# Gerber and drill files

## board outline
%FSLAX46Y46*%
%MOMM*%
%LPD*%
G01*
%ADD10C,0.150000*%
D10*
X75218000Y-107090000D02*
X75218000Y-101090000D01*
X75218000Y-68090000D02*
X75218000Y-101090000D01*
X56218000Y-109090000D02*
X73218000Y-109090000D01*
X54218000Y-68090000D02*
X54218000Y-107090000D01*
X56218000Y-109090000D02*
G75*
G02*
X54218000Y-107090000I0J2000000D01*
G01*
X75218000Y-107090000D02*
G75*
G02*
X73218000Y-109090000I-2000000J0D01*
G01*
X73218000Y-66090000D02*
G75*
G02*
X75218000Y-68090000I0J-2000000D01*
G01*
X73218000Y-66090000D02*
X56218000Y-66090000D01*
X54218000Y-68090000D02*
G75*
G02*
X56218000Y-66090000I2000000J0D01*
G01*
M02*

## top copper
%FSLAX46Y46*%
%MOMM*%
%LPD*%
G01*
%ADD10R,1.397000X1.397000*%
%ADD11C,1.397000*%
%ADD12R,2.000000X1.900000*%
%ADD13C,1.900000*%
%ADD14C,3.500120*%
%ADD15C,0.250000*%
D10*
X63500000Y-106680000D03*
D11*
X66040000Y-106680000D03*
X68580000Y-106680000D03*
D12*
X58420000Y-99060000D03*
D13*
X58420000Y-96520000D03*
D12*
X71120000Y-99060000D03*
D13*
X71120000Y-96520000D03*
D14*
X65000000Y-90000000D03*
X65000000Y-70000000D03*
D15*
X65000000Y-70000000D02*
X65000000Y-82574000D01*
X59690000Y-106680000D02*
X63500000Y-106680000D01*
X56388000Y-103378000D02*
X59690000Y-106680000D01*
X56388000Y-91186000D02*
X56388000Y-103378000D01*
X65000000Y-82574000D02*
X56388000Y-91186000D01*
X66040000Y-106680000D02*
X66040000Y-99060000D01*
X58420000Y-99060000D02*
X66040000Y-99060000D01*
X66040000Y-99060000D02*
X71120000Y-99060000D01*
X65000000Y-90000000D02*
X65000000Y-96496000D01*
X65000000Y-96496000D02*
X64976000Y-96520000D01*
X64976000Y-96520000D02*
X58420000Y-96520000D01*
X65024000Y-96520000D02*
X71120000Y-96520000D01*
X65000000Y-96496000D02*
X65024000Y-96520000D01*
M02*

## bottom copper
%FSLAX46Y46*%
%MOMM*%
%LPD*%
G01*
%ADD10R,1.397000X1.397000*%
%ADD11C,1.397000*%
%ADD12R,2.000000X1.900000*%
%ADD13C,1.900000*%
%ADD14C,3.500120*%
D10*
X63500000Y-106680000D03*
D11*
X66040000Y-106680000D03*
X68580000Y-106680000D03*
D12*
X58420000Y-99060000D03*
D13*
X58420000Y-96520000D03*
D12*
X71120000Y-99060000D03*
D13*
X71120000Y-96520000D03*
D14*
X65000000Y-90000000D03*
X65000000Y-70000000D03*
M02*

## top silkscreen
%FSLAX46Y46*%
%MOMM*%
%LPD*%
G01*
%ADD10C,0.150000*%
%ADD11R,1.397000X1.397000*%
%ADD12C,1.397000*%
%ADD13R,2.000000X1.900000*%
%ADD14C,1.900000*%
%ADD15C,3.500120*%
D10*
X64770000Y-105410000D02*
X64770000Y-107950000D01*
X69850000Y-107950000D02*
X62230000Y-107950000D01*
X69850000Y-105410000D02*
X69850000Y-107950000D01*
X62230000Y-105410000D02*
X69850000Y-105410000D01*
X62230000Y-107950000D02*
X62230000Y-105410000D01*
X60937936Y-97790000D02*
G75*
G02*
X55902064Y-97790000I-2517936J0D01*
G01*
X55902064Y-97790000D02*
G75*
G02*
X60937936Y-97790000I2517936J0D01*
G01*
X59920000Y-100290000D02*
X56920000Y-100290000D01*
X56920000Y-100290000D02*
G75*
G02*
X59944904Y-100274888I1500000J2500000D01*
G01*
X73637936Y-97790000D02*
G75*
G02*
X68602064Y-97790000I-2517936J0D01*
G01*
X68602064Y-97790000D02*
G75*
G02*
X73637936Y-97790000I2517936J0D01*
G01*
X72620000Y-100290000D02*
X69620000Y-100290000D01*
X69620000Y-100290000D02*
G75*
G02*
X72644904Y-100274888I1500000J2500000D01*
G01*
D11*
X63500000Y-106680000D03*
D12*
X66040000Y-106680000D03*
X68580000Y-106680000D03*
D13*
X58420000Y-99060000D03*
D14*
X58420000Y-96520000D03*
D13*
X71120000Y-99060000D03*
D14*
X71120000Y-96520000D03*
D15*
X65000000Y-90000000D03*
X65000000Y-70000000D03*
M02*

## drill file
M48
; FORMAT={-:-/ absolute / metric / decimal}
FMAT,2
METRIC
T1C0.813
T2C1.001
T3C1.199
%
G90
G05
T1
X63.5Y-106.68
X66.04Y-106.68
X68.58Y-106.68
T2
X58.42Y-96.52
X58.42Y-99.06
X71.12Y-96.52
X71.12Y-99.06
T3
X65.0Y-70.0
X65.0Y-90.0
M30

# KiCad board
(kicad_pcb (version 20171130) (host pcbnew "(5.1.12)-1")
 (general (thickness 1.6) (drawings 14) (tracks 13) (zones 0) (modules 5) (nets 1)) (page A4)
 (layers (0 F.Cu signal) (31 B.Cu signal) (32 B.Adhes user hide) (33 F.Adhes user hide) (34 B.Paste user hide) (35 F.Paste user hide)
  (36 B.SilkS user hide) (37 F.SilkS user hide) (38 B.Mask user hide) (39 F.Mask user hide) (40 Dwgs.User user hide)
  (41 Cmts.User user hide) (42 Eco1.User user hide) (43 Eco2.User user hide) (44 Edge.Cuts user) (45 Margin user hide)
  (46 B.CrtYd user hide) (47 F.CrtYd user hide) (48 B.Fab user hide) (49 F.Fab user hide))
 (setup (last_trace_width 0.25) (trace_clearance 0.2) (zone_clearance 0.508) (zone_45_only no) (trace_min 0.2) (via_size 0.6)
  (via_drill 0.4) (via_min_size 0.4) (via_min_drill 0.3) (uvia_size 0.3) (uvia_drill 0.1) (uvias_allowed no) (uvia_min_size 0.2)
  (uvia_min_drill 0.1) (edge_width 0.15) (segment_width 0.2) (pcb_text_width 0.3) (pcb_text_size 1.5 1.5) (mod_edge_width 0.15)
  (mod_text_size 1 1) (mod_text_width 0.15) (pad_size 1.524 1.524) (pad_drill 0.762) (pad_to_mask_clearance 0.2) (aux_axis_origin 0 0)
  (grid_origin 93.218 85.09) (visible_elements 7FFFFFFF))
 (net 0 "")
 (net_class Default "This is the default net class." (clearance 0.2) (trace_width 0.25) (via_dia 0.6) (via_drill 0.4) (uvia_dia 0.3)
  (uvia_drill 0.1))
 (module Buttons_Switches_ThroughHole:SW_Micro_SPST (layer F.Cu) (at 66.04 106.68)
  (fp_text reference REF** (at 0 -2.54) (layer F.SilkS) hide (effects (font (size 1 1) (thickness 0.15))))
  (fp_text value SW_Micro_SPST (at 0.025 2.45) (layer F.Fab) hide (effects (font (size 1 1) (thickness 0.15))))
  (fp_line (start -1.27 -1.27) (end -1.27 1.27) (layer F.SilkS) (width 0.15))
  (fp_line (start 3.81 1.27) (end -3.81 1.27) (layer F.SilkS) (width 0.15))
  (fp_line (start 3.81 -1.27) (end 3.81 1.27) (layer F.SilkS) (width 0.15))
  (fp_line (start -3.81 -1.27) (end 3.81 -1.27) (layer F.SilkS) (width 0.15))
  (fp_line (start -3.81 1.27) (end -3.81 -1.27) (layer F.SilkS) (width 0.15))
  (pad 1 thru_hole rect (at -2.54 0) (size 1.397 1.397) (drill 0.8128) (layers *.Cu *.Mask F.SilkS))
  (pad 2 thru_hole circle (at 0 0) (size 1.397 1.397) (drill 0.8128) (layers *.Cu *.Mask F.SilkS))
  (pad 3 thru_hole circle (at 2.54 0) (size 1.397 1.397) (drill 0.8128) (layers *.Cu *.Mask F.SilkS)))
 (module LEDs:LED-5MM (layer F.Cu) (at 58.42 99.06 90)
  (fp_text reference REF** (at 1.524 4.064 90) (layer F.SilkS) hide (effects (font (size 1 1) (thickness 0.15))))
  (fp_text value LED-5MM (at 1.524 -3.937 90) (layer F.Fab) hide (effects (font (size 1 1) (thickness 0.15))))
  (fp_circle (center 1.27 0) (end 0.97 -2.5) (layer F.SilkS) (width 0.15))
  (fp_line (start -1.23 1.5) (end -1.23 -1.5) (layer F.SilkS) (width 0.15))
  (fp_arc (start 1.27 0) (end -1.23 -1.5) (angle 297.5) (layer F.SilkS) (width 0.15))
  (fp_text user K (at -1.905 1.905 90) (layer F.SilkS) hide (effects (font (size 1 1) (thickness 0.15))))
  (pad 1 thru_hole rect (at 0 0 180) (size 2 1.9) (drill 1.00076) (layers *.Cu *.Mask F.SilkS))
  (pad 2 thru_hole circle (at 2.54 0 90) (size 1.9 1.9) (drill 1.00076) (layers *.Cu *.Mask F.SilkS)))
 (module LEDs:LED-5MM (layer F.Cu) (at 71.12 99.06 90)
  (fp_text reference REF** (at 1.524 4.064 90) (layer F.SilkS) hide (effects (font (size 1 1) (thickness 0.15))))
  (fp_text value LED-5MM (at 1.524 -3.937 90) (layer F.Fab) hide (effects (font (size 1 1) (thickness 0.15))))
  (fp_circle (center 1.27 0) (end 0.97 -2.5) (layer F.SilkS) (width 0.15))
  (fp_line (start -1.23 1.5) (end -1.23 -1.5) (layer F.SilkS) (width 0.15))
  (fp_arc (start 1.27 0) (end -1.23 -1.5) (angle 297.5) (layer F.SilkS) (width 0.15))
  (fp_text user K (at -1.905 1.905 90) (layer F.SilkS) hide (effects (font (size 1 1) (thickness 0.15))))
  (pad 1 thru_hole rect (at 0 0 180) (size 2 1.9) (drill 1.00076) (layers *.Cu *.Mask F.SilkS))
  (pad 2 thru_hole circle (at 2.54 0 90) (size 1.9 1.9) (drill 1.00076) (layers *.Cu *.Mask F.SilkS)))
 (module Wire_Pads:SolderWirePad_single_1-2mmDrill (layer F.Cu) (at 65 90)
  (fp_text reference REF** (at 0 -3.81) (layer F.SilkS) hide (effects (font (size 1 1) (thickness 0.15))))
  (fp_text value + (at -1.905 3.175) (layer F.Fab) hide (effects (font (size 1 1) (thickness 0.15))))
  (pad 1 thru_hole circle (at 0 0) (size 3.50012 3.50012) (drill 1.19888) (layers *.Cu *.Mask F.SilkS)))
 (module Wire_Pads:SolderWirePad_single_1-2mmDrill (layer F.Cu) (at 65 70)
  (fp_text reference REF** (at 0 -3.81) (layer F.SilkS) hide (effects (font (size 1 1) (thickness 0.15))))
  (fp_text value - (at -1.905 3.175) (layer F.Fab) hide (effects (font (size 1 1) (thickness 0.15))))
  (pad 1 thru_hole circle (at 0 0) (size 3.50012 3.50012) (drill 1.19888) (layers *.Cu *.Mask F.SilkS)))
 (gr_line (start 75.218 107.09) (end 75.218 101.09) (angle 90) (layer Edge.Cuts) (width 0.15))
 (gr_line (start 75.218 68.09) (end 75.218 101.09) (angle 90) (layer Edge.Cuts) (width 0.15))
 (gr_line (start 56.218 109.09) (end 73.218 109.09) (angle 90) (layer Edge.Cuts) (width 0.15))
 (gr_line (start 54.218 68.09) (end 54.218 107.09) (angle 90) (layer Edge.Cuts) (width 0.15))
 (gr_arc (start 56.218 107.09) (end 56.218 109.09) (angle 90) (layer Edge.Cuts) (width 0.15))
 (gr_arc (start 73.218 107.09) (end 75.218 107.09) (angle 90) (layer Edge.Cuts) (width 0.15))
 (gr_arc (start 73.218 68.09) (end 73.218 66.09) (angle 90) (layer Edge.Cuts) (width 0.15))
 (gr_line (start 73.218 66.09) (end 56.218 66.09) (angle 90) (layer Edge.Cuts) (width 0.15))
 (gr_arc (start 56.218 68.09) (end 54.218 68.09) (angle 90) (layer Edge.Cuts) (width 0.15))
 (segment (start 65 70) (end 65 82.574) (width 0.25) (layer F.Cu) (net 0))
 (segment (start 59.69 106.68) (end 63.5 106.68) (width 0.25) (layer F.Cu) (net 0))
 (segment (start 56.388 103.378) (end 59.69 106.68) (width 0.25) (layer F.Cu) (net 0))
 (segment (start 56.388 91.186) (end 56.388 103.378) (width 0.25) (layer F.Cu) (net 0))
 (segment (start 65 82.574) (end 56.388 91.186) (width 0.25) (layer F.Cu) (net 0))
 (segment (start 66.04 106.68) (end 66.04 99.06) (width 0.25) (layer F.Cu) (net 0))
 (segment (start 58.42 99.06) (end 66.04 99.06) (width 0.25) (layer F.Cu) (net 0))
 (segment (start 66.04 99.06) (end 71.12 99.06) (width 0.25) (layer F.Cu) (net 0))
 (segment (start 65 90) (end 65 96.496) (width 0.25) (layer F.Cu) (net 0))
 (segment (start 65 96.496) (end 64.976 96.52) (width 0.25) (layer F.Cu) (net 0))
 (segment (start 64.976 96.52) (end 58.42 96.52) (width 0.25) (layer F.Cu) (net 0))
 (segment (start 65.024 96.52) (end 71.12 96.52) (width 0.25) (layer F.Cu) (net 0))
 (segment (start 65 96.496) (end 65.024 96.52) (width 0.25) (layer F.Cu) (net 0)))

